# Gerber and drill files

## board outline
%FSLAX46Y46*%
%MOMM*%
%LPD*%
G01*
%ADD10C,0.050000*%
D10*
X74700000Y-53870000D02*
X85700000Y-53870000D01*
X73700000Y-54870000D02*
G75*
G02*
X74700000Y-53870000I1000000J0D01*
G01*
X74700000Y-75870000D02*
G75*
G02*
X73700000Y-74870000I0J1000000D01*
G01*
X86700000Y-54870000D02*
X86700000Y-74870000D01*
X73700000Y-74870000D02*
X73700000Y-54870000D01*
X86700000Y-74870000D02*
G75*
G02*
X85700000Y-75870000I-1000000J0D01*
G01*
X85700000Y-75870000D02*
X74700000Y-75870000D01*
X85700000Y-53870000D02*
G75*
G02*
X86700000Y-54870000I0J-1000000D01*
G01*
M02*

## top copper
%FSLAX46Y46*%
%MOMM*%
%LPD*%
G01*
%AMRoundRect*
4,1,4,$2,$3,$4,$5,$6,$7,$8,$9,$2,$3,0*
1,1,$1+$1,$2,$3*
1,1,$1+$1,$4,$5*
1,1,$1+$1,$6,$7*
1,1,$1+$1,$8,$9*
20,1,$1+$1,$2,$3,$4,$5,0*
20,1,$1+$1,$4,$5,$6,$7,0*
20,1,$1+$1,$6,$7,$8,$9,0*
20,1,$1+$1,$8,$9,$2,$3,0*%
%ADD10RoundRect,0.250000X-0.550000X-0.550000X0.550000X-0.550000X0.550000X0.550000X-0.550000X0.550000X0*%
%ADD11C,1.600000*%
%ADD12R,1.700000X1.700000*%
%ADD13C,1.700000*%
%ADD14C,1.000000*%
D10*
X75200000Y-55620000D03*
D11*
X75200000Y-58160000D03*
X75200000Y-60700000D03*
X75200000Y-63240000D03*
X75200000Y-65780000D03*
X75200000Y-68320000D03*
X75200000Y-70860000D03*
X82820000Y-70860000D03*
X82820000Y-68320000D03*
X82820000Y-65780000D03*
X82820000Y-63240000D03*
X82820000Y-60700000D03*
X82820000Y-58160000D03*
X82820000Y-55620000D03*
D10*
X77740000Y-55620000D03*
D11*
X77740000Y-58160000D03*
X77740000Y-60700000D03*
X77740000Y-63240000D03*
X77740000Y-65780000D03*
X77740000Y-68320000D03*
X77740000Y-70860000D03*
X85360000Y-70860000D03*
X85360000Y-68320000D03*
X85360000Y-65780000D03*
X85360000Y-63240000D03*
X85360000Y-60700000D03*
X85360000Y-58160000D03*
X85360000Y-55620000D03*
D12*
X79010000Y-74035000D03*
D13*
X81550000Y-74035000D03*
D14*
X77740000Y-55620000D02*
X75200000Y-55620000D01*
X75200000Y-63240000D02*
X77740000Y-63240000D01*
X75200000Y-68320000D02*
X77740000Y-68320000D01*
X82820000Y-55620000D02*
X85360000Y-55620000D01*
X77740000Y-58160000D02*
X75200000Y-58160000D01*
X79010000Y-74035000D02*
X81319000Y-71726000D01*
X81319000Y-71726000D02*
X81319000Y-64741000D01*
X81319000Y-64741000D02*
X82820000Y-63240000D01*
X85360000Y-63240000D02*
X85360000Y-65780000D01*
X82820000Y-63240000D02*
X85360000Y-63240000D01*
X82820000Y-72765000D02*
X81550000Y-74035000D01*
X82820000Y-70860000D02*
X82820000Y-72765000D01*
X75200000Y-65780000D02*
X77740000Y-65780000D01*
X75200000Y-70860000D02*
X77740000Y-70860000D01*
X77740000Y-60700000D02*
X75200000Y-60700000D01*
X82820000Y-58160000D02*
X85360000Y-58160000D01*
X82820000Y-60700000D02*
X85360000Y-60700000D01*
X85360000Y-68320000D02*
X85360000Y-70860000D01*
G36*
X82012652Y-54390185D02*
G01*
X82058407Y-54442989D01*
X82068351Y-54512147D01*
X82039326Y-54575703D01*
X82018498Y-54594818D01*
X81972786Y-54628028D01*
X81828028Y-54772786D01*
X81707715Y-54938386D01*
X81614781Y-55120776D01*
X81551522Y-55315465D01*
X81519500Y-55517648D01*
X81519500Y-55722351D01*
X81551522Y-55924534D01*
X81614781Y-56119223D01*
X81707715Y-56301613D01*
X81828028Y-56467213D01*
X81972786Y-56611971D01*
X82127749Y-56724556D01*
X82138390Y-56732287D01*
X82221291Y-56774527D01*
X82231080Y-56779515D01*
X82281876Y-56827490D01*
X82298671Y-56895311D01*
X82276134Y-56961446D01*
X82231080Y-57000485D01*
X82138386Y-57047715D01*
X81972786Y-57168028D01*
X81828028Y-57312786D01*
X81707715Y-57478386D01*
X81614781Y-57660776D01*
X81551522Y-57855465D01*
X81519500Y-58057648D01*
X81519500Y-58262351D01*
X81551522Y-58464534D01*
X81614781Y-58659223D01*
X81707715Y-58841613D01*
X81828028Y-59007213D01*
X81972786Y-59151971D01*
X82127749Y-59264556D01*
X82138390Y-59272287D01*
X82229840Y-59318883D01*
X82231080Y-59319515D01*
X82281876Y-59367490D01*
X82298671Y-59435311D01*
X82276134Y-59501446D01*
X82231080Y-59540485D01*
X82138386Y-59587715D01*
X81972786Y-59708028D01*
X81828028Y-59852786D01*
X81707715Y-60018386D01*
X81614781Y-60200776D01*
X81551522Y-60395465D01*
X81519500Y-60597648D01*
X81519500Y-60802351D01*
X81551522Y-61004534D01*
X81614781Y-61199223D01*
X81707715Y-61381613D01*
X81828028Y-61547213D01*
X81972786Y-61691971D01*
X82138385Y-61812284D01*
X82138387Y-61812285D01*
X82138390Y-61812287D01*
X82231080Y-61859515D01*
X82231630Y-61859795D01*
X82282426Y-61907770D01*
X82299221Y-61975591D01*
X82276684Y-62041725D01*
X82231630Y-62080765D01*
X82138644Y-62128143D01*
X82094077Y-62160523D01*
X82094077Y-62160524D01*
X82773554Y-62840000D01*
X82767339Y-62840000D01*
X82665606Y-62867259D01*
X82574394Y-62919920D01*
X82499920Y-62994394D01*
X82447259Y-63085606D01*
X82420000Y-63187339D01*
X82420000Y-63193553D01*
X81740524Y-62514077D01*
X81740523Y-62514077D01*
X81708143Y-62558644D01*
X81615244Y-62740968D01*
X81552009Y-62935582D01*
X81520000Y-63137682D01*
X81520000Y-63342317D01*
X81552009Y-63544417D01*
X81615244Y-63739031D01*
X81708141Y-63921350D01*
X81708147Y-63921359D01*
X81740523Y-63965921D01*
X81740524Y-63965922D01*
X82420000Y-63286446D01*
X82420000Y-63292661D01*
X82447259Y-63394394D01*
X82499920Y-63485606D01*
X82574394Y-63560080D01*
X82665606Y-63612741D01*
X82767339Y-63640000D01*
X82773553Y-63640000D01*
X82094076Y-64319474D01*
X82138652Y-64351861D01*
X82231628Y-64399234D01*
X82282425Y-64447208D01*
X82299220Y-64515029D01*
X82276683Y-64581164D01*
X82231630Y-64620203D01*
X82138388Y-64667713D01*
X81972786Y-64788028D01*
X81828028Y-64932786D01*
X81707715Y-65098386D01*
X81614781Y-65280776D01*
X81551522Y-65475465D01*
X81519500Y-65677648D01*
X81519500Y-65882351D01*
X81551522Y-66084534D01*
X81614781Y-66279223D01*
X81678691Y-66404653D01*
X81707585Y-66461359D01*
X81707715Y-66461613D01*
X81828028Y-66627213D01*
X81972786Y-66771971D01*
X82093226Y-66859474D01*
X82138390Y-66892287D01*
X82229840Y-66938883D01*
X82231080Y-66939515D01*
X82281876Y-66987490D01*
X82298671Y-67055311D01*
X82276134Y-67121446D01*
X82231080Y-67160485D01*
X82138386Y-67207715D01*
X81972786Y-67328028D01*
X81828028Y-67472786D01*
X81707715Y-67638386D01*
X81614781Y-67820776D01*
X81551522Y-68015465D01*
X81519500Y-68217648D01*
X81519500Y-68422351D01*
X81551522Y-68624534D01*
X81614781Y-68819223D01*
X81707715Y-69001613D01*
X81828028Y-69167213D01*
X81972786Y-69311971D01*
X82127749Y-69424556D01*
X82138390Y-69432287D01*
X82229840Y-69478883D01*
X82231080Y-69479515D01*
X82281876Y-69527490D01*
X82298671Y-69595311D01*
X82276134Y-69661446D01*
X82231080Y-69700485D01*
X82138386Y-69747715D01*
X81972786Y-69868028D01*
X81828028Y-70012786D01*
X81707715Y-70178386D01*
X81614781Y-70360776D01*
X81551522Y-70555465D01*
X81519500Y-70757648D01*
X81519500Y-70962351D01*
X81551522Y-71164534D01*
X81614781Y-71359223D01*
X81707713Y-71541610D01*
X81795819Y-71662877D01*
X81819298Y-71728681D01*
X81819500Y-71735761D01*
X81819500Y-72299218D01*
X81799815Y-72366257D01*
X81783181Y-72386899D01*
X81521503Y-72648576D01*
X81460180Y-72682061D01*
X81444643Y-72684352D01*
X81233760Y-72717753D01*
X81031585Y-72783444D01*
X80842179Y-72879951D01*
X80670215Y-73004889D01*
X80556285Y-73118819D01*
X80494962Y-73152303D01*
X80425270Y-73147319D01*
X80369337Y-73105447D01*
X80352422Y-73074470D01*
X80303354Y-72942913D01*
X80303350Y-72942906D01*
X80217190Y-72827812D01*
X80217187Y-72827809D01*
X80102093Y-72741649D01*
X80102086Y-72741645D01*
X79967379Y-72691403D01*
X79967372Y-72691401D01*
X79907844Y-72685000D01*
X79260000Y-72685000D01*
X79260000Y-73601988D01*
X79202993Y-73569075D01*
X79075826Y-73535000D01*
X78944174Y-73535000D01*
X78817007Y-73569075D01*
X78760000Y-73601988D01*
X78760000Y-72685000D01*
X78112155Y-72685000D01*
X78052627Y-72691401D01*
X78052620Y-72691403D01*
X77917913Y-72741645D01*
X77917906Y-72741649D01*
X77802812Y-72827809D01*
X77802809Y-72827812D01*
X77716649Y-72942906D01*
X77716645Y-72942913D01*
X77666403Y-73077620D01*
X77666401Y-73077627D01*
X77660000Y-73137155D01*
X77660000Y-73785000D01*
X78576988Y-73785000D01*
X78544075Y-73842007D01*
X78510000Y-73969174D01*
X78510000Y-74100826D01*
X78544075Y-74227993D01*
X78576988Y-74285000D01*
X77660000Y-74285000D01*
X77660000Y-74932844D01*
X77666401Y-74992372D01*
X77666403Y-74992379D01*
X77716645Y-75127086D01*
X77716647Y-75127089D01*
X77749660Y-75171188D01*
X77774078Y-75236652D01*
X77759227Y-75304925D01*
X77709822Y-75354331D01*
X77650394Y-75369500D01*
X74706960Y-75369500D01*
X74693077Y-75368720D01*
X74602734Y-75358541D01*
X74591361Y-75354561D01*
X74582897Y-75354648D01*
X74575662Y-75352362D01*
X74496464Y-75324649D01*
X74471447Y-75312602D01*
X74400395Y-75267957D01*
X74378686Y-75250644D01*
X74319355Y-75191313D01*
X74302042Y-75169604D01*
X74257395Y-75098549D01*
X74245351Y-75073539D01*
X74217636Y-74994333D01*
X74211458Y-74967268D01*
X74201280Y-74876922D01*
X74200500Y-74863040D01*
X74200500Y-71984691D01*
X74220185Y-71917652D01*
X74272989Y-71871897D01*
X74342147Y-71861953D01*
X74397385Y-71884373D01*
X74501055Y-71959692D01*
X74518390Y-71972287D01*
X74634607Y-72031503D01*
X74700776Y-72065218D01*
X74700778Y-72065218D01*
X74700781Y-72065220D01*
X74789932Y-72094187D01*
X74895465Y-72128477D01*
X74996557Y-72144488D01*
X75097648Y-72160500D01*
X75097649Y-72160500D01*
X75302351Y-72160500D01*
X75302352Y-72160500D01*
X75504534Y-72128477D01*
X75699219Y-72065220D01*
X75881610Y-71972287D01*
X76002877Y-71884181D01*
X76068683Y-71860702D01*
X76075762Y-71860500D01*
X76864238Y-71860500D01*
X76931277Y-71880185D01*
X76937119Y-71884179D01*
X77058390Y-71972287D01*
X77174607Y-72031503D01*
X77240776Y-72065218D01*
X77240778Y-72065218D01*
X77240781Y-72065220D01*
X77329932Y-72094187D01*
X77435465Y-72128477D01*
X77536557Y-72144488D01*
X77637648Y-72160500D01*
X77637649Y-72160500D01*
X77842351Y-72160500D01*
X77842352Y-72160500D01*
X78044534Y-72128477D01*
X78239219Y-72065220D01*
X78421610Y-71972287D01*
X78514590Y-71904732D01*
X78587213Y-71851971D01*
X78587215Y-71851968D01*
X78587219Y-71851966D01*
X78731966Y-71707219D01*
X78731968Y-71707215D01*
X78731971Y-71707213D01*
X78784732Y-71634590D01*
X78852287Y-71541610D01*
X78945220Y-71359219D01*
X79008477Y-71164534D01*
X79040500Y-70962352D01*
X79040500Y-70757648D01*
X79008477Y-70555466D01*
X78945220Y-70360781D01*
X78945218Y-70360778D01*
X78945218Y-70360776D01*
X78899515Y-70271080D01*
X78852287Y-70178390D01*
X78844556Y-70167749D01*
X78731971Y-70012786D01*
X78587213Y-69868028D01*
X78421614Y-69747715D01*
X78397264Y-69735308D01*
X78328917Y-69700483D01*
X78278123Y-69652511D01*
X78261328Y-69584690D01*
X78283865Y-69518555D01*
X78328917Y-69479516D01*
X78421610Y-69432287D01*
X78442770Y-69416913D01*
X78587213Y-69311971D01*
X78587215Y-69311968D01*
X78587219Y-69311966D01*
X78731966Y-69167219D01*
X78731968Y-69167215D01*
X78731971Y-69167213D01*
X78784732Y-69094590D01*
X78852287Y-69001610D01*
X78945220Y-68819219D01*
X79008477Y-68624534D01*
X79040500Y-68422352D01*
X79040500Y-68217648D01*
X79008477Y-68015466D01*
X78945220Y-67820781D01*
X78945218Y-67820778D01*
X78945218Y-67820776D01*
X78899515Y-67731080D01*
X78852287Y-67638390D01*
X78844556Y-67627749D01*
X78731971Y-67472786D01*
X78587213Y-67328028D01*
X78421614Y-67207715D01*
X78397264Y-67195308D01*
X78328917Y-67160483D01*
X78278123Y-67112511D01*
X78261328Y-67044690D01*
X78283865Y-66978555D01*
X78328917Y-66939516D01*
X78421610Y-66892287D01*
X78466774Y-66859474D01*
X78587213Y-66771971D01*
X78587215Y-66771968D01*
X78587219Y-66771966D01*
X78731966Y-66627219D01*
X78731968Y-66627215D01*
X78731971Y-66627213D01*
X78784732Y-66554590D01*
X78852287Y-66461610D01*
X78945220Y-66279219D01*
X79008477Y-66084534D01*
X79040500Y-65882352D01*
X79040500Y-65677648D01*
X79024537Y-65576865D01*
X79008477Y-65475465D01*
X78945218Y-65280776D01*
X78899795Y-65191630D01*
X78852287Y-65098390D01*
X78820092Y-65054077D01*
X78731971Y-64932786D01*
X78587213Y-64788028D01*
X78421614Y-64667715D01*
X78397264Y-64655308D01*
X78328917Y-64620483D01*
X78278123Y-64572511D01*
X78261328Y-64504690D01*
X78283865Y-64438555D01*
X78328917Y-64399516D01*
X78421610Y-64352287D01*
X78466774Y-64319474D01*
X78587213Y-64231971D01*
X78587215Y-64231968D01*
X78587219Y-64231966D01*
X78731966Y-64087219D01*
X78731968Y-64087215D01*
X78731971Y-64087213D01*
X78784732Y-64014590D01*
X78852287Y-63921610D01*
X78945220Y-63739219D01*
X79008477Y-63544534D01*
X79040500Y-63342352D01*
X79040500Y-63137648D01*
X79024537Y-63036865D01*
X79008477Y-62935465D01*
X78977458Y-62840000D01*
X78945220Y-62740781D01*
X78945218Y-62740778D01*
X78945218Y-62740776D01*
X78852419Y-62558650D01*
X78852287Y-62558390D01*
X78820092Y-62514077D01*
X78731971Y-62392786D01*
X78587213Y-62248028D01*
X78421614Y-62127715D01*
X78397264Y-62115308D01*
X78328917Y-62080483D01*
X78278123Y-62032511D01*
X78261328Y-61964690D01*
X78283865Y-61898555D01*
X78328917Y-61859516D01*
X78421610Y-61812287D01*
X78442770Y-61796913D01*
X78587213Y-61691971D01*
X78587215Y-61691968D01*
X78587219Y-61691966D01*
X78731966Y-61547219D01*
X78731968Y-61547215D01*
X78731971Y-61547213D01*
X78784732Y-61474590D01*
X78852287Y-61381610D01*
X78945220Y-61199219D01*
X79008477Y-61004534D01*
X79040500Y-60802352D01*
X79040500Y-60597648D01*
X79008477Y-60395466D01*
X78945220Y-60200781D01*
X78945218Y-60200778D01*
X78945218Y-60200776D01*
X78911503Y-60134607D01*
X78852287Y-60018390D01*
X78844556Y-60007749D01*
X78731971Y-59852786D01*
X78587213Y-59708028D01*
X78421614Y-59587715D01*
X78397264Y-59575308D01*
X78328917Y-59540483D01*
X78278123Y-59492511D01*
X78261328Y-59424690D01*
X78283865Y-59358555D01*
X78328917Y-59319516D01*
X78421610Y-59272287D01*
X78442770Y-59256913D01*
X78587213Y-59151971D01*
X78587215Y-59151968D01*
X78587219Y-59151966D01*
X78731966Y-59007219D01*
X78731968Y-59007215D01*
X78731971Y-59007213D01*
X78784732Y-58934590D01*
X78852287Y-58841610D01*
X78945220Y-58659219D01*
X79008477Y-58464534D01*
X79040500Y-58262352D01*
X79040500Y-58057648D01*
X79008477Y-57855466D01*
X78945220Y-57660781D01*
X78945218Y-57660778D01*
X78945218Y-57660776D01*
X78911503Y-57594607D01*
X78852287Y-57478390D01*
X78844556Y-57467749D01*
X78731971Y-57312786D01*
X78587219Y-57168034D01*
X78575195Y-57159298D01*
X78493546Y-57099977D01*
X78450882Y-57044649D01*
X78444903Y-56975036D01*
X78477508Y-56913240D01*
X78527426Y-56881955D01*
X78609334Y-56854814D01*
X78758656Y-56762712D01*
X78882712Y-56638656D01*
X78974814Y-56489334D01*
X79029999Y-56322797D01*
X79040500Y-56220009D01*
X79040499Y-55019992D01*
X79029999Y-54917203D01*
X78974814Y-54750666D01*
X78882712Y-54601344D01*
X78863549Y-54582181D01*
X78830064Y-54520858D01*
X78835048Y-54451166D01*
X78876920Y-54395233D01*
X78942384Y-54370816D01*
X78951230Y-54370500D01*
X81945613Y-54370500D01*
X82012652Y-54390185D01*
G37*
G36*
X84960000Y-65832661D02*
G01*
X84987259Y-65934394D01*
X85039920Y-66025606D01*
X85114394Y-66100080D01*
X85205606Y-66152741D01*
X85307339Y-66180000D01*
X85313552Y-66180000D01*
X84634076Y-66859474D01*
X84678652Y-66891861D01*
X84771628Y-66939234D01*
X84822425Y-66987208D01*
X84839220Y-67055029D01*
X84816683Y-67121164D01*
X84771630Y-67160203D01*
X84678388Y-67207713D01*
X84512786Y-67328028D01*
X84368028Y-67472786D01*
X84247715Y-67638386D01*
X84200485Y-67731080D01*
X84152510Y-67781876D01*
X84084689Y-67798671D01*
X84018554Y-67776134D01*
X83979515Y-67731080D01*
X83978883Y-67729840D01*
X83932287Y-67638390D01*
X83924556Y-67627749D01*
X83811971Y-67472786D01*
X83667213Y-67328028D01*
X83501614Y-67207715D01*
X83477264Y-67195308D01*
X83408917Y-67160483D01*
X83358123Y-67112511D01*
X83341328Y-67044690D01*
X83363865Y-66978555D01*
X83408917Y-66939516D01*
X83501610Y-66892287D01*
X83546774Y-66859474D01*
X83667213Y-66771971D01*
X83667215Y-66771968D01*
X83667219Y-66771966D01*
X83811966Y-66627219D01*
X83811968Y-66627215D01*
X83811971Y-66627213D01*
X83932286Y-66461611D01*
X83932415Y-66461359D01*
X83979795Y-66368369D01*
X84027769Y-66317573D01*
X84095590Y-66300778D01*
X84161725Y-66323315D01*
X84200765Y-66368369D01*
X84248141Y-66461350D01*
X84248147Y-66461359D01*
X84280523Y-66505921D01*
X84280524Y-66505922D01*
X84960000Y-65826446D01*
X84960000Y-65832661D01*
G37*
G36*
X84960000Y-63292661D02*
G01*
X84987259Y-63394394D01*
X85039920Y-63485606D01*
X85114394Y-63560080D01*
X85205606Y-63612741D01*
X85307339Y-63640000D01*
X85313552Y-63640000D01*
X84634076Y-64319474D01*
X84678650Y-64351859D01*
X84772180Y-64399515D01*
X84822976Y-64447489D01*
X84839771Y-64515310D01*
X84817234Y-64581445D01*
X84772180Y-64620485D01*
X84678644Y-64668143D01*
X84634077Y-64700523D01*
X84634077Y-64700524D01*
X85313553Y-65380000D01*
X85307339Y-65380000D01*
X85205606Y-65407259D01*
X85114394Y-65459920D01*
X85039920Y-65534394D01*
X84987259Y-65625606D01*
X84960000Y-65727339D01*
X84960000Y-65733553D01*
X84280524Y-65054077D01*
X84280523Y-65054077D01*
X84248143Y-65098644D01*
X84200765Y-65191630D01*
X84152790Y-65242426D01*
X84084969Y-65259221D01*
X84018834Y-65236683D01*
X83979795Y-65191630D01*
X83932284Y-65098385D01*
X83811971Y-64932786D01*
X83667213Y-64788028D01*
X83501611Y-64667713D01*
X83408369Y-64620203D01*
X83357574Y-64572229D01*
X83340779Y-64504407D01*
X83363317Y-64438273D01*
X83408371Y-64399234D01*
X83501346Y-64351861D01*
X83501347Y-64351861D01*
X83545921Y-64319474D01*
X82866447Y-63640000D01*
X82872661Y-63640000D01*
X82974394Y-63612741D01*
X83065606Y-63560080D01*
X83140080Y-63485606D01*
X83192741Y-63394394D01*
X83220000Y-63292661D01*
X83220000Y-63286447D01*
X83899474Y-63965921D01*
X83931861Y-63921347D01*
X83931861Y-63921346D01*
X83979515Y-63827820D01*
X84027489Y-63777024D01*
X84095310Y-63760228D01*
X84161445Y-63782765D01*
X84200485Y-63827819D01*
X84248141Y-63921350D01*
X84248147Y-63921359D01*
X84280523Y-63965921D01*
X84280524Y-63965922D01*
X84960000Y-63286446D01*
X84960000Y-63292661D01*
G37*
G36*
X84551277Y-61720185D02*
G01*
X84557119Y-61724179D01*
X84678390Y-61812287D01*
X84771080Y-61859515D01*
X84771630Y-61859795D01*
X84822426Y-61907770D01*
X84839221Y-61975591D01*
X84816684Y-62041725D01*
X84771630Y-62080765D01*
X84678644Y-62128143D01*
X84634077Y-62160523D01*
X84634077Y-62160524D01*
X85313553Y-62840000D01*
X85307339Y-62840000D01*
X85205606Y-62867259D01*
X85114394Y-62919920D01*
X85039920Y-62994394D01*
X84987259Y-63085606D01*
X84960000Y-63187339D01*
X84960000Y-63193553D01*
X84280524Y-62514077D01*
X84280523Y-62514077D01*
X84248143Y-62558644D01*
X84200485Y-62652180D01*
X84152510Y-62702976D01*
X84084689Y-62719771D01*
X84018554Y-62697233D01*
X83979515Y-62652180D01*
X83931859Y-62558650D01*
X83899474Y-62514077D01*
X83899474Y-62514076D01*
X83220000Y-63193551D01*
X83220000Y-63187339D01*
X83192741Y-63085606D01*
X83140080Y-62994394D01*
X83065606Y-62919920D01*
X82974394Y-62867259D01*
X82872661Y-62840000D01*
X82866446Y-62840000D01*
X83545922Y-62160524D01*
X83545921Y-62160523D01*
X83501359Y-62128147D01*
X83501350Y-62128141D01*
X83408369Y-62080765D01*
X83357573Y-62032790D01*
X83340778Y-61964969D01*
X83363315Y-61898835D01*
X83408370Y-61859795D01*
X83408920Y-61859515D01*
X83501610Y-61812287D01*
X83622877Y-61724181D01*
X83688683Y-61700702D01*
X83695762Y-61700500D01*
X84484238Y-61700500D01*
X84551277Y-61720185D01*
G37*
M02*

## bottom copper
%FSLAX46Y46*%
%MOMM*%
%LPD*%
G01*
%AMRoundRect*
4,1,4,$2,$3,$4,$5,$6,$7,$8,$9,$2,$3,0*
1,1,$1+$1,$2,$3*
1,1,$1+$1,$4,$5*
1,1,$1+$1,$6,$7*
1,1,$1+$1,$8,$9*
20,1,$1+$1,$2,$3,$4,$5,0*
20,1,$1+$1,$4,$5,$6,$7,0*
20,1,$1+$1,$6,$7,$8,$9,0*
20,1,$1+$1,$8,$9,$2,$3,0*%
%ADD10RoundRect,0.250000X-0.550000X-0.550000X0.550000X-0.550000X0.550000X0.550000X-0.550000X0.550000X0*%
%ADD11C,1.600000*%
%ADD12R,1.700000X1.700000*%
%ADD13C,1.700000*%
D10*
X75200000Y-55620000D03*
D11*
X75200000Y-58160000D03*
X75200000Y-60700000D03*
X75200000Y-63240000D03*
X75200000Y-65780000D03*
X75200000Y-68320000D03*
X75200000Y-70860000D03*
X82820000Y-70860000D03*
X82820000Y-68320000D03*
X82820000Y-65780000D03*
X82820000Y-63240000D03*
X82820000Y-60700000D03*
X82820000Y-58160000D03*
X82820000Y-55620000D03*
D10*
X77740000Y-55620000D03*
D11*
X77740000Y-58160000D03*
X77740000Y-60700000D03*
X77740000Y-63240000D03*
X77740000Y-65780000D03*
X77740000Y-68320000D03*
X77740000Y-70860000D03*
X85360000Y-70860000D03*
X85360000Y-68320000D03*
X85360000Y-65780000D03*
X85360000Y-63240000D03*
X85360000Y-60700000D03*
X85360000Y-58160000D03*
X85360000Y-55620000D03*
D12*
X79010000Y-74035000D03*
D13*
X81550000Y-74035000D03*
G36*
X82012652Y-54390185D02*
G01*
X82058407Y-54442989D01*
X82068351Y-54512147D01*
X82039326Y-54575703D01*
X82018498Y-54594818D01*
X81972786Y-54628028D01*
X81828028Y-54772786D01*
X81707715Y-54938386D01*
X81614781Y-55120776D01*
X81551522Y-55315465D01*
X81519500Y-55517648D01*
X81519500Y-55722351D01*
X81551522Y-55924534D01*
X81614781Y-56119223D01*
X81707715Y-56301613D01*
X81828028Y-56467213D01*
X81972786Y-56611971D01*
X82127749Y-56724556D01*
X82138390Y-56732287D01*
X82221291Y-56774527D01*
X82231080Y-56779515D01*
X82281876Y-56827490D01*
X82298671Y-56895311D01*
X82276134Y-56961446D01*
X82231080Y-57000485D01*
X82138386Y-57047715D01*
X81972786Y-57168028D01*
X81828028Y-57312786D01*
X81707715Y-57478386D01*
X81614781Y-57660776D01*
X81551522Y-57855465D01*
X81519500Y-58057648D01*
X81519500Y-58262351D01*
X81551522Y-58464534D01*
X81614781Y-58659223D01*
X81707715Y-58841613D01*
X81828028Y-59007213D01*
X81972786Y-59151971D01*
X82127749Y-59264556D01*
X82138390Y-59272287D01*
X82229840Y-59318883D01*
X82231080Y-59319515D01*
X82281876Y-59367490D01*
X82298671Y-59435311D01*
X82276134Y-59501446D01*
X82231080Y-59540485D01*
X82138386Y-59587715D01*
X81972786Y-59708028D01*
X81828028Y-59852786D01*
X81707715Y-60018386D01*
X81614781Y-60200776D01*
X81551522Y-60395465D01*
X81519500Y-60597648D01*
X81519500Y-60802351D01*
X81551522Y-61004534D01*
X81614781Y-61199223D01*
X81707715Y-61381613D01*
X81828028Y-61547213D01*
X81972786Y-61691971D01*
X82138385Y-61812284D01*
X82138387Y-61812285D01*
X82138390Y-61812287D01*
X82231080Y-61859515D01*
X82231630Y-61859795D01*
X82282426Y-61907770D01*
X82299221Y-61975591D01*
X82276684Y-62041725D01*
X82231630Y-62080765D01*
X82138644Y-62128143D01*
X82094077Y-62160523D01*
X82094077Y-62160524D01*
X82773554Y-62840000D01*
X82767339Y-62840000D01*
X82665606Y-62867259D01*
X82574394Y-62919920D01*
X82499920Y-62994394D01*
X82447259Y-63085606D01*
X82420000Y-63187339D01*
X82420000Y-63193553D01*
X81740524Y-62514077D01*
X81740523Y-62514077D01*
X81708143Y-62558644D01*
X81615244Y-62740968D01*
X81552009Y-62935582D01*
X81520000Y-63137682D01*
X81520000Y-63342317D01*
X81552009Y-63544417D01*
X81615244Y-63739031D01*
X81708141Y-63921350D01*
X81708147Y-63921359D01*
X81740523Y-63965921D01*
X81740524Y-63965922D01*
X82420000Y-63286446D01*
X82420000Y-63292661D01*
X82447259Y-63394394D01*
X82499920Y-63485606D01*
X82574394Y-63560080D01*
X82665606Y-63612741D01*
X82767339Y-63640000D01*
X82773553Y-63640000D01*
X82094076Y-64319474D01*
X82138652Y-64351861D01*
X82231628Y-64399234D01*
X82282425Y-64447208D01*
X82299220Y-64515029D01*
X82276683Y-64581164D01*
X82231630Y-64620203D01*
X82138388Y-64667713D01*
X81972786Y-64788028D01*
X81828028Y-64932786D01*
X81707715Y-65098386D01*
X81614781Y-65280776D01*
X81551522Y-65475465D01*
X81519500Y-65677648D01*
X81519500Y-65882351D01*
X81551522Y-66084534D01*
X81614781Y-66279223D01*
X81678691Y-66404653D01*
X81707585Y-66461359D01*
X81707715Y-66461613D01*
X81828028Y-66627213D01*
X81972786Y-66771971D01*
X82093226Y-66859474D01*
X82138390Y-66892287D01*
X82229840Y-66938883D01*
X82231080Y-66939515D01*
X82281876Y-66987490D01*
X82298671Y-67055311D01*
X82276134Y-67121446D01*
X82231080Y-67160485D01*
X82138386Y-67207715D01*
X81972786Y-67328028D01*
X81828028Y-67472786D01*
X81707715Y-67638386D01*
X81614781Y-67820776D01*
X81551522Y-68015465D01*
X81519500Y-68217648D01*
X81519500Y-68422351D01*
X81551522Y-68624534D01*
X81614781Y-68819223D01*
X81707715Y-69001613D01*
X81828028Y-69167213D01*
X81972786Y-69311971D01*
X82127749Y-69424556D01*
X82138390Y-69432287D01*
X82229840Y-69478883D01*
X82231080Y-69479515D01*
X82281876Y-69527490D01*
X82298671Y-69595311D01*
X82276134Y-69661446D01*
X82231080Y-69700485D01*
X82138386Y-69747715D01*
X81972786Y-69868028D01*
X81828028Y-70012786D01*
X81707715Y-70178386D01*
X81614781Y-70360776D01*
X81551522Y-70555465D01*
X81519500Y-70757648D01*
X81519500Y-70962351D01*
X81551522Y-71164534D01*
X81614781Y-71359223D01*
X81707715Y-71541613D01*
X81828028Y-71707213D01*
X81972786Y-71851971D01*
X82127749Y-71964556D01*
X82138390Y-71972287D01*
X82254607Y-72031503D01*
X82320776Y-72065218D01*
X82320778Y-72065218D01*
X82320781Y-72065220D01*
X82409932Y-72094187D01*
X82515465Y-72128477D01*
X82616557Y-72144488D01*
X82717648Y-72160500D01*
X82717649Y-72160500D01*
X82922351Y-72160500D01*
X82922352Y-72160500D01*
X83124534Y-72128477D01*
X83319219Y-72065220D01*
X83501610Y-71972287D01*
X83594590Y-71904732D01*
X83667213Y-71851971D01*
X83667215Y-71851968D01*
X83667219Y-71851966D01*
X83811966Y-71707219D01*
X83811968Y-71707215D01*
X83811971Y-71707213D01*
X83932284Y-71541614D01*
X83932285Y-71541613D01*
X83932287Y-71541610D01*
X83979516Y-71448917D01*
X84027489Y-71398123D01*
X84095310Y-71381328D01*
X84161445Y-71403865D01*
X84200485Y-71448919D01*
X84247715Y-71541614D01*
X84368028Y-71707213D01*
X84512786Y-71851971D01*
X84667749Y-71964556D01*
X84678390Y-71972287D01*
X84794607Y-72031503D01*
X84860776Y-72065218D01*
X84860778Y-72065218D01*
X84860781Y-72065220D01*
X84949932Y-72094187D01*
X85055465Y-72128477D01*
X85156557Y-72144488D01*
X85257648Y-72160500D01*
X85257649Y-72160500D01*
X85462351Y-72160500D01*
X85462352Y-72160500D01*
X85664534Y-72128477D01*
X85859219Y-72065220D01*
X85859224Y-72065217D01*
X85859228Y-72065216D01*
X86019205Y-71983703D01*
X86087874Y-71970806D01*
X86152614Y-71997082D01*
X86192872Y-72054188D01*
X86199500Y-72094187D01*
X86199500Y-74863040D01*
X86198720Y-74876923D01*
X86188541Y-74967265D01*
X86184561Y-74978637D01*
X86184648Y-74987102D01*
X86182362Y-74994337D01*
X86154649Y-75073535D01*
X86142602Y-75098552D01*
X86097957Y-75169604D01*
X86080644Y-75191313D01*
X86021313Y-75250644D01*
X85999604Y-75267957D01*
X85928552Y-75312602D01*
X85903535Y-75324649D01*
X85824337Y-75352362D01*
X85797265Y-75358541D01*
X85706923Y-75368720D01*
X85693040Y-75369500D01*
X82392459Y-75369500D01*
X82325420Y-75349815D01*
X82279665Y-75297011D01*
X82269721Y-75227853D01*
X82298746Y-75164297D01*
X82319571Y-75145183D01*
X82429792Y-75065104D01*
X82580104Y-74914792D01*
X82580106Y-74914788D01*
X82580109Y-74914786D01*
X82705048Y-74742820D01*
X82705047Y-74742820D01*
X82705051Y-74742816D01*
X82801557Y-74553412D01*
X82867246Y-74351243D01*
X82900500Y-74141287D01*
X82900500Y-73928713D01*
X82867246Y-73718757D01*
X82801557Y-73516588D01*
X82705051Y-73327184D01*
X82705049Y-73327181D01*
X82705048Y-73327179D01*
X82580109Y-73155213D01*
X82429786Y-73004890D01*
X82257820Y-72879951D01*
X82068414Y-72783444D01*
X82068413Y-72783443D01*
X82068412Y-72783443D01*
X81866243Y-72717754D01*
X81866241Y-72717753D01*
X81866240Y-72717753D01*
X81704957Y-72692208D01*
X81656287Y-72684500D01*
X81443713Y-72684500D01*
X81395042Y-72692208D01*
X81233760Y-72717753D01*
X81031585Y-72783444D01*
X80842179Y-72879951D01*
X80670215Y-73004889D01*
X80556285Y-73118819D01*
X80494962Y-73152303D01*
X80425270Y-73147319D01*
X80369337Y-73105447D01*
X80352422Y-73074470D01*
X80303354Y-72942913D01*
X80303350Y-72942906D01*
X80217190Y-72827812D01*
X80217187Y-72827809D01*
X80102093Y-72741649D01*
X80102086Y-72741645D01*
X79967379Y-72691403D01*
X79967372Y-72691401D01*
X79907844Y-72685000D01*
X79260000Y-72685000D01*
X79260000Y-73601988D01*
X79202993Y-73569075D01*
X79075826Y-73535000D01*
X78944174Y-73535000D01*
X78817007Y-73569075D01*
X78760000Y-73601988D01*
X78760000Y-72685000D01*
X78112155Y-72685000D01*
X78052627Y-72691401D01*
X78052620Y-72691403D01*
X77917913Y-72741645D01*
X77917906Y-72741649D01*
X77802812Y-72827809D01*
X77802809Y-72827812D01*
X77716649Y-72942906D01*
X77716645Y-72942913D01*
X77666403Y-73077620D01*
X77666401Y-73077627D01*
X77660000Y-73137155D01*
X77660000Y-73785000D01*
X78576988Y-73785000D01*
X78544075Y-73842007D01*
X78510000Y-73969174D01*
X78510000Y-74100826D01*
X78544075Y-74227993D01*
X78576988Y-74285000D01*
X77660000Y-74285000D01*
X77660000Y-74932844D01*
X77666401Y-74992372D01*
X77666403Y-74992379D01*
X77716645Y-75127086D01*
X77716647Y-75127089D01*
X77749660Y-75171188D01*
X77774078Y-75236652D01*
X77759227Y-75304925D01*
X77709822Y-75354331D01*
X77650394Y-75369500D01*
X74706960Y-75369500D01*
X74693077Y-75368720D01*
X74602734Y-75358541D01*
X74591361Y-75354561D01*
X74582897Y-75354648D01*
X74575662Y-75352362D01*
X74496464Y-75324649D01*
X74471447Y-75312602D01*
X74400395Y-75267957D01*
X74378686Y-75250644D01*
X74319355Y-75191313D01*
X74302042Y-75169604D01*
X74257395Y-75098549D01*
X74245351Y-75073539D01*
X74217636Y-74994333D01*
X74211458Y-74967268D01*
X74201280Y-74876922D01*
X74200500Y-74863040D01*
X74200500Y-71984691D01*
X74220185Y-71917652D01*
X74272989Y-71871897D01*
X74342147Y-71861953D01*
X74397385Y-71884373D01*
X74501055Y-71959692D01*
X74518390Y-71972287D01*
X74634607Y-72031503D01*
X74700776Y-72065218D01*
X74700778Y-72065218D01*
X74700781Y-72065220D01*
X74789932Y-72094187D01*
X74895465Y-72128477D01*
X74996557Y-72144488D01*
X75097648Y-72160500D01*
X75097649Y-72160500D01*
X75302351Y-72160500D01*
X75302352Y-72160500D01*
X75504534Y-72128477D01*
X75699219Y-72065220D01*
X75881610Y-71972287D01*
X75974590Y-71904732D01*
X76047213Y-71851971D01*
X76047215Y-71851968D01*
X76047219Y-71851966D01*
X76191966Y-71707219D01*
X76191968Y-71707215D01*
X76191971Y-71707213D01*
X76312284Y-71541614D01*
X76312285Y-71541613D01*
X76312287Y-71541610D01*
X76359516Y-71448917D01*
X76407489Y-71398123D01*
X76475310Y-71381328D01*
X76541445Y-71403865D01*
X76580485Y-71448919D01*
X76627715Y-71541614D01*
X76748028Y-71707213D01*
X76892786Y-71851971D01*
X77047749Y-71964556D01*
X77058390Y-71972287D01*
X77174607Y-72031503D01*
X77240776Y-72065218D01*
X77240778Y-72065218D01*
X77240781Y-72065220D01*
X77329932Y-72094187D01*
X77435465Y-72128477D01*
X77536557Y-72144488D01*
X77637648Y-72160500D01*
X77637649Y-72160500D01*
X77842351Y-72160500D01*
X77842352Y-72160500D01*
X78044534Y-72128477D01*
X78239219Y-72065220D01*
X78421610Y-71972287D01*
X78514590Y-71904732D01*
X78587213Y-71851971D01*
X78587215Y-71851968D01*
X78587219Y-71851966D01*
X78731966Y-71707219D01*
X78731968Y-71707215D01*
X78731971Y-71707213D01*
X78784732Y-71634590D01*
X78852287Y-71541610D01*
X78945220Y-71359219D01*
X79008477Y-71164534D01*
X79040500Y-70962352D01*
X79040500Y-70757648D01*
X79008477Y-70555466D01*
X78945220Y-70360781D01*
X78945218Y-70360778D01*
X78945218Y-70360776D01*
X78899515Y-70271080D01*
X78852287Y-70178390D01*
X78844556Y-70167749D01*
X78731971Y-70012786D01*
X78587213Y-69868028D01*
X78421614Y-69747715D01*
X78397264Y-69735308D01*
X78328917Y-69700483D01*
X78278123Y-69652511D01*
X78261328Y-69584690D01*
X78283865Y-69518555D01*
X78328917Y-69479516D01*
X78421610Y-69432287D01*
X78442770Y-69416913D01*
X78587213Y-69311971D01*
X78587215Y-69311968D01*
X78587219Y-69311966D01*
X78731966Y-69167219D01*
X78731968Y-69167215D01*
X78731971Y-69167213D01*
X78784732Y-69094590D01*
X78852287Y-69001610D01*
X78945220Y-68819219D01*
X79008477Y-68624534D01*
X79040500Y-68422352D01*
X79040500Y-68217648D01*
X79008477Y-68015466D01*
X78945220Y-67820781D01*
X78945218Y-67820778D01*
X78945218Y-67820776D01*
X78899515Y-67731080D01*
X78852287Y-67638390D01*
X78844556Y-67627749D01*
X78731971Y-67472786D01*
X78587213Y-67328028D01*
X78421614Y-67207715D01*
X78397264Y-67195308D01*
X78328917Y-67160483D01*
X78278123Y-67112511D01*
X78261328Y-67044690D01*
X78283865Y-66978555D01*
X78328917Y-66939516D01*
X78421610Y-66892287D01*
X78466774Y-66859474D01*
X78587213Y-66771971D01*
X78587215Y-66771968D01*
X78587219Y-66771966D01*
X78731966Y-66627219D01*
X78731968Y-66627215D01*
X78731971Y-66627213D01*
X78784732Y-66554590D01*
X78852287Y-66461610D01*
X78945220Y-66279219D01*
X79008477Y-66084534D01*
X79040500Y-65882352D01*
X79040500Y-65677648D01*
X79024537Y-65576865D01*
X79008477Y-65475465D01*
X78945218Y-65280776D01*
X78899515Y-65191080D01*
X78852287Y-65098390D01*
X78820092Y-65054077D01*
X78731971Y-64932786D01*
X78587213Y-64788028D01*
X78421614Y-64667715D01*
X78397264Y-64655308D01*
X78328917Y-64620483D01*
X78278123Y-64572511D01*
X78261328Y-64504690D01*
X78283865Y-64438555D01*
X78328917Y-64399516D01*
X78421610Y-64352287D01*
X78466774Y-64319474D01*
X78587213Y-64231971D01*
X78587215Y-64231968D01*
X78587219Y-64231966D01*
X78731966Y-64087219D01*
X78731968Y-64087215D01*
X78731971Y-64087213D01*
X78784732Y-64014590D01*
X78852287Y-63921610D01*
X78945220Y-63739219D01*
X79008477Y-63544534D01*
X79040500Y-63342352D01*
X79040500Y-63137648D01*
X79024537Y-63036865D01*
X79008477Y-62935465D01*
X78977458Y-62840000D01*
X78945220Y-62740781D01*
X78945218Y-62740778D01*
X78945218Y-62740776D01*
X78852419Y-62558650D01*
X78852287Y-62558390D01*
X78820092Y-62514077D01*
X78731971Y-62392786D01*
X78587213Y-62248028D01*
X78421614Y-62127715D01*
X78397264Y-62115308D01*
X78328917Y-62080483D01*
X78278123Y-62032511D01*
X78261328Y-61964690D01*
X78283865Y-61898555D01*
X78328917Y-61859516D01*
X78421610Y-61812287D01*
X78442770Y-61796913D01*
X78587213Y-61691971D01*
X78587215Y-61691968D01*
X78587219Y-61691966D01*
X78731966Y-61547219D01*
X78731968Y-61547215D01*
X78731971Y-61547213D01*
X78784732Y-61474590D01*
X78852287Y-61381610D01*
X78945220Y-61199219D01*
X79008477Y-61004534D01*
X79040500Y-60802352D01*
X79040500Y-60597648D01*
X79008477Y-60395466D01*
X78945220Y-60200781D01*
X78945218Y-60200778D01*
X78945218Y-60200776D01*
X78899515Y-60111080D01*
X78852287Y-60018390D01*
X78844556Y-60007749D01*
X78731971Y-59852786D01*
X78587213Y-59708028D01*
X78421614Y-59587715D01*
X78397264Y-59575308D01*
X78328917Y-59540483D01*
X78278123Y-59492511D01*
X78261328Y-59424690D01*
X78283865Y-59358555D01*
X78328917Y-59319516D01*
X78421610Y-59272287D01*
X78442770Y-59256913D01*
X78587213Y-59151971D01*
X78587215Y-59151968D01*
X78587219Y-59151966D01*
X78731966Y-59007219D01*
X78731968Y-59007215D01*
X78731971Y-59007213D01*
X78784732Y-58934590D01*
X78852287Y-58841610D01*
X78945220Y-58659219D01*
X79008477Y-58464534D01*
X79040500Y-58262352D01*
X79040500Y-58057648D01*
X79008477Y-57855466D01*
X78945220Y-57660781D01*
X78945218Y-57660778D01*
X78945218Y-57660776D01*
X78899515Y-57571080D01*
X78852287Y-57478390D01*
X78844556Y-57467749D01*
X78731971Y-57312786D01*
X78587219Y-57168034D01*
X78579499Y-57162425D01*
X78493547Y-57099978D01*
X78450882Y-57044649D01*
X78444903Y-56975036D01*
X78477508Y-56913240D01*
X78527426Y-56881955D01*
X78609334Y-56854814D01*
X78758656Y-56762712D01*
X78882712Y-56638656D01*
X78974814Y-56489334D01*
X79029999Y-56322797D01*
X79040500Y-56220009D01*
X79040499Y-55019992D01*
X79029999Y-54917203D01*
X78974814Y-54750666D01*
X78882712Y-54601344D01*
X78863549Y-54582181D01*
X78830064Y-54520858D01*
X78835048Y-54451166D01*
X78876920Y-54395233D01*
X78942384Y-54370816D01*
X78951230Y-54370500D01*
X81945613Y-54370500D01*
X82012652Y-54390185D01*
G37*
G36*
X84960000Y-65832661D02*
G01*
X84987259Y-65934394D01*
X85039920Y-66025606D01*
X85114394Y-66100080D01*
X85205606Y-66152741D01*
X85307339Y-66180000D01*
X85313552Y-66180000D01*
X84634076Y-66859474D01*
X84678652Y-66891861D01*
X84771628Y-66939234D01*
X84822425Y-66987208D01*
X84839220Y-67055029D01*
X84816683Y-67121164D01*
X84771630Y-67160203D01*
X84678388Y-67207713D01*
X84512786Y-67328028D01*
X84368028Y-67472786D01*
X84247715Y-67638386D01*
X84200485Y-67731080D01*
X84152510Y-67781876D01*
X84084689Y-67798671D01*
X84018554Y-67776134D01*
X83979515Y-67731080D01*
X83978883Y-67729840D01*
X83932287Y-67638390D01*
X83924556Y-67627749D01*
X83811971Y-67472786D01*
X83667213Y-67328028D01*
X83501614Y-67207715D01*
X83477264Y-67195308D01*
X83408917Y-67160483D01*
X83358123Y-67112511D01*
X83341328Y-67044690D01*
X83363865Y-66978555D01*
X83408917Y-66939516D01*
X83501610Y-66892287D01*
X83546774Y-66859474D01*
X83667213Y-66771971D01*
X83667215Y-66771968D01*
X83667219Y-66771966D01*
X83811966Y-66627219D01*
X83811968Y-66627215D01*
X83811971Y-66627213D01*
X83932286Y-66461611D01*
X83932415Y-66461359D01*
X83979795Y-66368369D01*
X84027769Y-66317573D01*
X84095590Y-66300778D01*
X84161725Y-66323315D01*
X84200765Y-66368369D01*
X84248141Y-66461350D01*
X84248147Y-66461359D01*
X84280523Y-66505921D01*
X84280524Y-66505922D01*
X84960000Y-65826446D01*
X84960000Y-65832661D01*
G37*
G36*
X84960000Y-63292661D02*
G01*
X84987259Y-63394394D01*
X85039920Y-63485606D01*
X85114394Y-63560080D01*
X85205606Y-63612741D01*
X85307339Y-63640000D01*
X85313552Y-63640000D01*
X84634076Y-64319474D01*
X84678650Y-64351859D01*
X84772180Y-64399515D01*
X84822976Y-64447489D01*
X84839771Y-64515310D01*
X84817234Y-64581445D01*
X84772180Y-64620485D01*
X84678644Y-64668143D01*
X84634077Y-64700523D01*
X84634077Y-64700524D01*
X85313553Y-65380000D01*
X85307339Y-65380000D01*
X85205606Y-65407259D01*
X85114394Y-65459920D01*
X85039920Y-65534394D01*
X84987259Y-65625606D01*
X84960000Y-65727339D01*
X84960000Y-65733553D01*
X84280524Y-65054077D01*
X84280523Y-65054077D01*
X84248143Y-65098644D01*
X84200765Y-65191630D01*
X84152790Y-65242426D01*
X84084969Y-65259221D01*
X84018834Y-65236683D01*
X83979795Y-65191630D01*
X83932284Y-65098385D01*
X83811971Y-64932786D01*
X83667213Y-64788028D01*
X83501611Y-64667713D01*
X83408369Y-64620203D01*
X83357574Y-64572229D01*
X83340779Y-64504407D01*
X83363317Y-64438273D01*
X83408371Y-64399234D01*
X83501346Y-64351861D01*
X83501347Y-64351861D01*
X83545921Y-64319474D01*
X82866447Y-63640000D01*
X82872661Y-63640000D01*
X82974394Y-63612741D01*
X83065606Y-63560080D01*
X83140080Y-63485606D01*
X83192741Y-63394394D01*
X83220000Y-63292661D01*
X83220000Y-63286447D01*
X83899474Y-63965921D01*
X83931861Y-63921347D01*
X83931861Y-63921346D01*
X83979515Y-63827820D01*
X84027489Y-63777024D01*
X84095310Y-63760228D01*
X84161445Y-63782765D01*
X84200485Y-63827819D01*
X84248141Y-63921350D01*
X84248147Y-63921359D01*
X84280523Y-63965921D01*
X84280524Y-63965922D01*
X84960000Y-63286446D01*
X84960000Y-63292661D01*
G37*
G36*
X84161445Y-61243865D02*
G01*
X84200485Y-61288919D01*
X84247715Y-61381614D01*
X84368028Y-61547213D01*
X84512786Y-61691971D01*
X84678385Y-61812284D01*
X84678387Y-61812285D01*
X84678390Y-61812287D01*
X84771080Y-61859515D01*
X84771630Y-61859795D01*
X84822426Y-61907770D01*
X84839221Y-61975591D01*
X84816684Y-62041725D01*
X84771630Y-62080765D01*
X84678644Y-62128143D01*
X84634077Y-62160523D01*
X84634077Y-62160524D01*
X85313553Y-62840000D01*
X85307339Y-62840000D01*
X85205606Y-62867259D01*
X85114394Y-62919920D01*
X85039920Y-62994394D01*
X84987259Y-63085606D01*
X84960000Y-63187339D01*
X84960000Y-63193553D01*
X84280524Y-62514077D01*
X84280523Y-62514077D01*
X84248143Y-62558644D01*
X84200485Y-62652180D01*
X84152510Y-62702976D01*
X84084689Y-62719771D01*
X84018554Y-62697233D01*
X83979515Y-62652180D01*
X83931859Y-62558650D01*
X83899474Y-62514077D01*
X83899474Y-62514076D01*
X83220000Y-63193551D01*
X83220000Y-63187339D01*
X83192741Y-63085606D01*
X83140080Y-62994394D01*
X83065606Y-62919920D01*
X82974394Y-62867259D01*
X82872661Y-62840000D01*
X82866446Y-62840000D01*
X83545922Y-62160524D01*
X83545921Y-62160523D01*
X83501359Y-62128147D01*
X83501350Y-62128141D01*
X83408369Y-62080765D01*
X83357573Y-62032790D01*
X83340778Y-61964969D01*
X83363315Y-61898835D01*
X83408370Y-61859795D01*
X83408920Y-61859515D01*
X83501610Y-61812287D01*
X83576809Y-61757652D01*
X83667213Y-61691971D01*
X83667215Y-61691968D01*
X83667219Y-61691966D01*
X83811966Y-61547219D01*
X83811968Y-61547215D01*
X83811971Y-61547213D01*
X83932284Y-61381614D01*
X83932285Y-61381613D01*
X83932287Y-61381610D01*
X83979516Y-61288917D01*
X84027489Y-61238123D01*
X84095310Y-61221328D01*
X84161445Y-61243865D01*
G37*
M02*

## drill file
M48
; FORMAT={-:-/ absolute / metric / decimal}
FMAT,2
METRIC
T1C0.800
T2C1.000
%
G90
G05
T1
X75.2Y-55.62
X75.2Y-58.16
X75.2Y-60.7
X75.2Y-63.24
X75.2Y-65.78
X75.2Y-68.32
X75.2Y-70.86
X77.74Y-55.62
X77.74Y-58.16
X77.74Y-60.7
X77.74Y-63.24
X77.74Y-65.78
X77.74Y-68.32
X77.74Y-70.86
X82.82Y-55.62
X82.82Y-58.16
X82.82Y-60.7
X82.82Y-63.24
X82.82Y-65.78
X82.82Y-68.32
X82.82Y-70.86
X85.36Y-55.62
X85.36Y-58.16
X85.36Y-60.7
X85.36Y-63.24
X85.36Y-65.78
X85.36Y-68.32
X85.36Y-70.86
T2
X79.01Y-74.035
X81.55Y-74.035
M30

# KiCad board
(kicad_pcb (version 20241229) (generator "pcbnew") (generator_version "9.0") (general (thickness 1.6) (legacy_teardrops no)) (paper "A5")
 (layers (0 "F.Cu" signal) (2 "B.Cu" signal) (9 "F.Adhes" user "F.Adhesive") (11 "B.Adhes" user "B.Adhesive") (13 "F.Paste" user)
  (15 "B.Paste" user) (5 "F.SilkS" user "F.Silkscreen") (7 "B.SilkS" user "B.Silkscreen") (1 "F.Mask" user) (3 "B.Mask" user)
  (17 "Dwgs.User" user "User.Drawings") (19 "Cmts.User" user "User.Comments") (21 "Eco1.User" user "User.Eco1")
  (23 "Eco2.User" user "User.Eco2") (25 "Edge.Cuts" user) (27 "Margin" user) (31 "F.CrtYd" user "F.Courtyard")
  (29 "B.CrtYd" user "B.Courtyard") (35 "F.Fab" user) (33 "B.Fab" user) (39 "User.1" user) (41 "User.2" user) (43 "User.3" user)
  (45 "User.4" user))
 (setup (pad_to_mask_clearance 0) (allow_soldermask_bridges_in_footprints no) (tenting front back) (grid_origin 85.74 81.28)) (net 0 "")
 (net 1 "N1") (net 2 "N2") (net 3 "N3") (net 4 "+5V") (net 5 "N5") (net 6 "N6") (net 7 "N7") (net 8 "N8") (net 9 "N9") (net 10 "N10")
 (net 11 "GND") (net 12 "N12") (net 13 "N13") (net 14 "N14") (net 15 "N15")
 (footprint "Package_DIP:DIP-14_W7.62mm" (layer "F.Cu") (at 75.2 55.62)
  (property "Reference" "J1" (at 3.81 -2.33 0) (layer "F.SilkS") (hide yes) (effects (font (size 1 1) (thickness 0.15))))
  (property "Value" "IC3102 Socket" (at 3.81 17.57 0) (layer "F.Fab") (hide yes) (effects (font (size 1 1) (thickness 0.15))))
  (pad "1" thru_hole roundrect (at 0 0) (size 1.6 1.6) (drill 0.8) (layers "*.Cu" "*.Mask") (remove_unused_layers no)
   (roundrect_rratio 0.15625) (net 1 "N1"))
  (pad "2" thru_hole circle (at 0 2.54) (size 1.6 1.6) (drill 0.8) (layers "*.Cu" "*.Mask") (remove_unused_layers no) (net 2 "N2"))
  (pad "3" thru_hole circle (at 0 5.08) (size 1.6 1.6) (drill 0.8) (layers "*.Cu" "*.Mask") (remove_unused_layers no) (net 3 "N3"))
  (pad "4" thru_hole circle (at 0 7.62) (size 1.6 1.6) (drill 0.8) (layers "*.Cu" "*.Mask") (remove_unused_layers no) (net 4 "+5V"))
  (pad "5" thru_hole circle (at 0 10.16) (size 1.6 1.6) (drill 0.8) (layers "*.Cu" "*.Mask") (remove_unused_layers no) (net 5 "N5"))
  (pad "6" thru_hole circle (at 0 12.7) (size 1.6 1.6) (drill 0.8) (layers "*.Cu" "*.Mask") (remove_unused_layers no) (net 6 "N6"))
  (pad "7" thru_hole circle (at 0 15.24) (size 1.6 1.6) (drill 0.8) (layers "*.Cu" "*.Mask") (remove_unused_layers no) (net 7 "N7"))
  (pad "8" thru_hole circle (at 7.62 15.24) (size 1.6 1.6) (drill 0.8) (layers "*.Cu" "*.Mask") (remove_unused_layers no) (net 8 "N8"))
  (pad "9" thru_hole circle (at 7.62 12.7) (size 1.6 1.6) (drill 0.8) (layers "*.Cu" "*.Mask") (remove_unused_layers no) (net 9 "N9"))
  (pad "10" thru_hole circle (at 7.62 10.16) (size 1.6 1.6) (drill 0.8) (layers "*.Cu" "*.Mask") (remove_unused_layers no) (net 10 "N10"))
  (pad "11" thru_hole circle (at 7.62 7.62) (size 1.6 1.6) (drill 0.8) (layers "*.Cu" "*.Mask") (remove_unused_layers no) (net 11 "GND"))
  (pad "12" thru_hole circle (at 7.62 5.08) (size 1.6 1.6) (drill 0.8) (layers "*.Cu" "*.Mask") (remove_unused_layers no) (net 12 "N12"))
  (pad "13" thru_hole circle (at 7.62 2.54) (size 1.6 1.6) (drill 0.8) (layers "*.Cu" "*.Mask") (remove_unused_layers no) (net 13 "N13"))
  (pad "14" thru_hole circle (at 7.62 0) (size 1.6 1.6) (drill 0.8) (layers "*.Cu" "*.Mask") (remove_unused_layers no) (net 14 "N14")))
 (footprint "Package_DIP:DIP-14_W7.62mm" (layer "F.Cu") (at 77.74 55.62)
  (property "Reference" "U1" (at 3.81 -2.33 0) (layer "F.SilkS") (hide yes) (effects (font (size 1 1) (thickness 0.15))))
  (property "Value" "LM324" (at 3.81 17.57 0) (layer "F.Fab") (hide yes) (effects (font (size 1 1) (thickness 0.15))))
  (pad "1" thru_hole roundrect (at 0 0) (size 1.6 1.6) (drill 0.8) (layers "*.Cu" "*.Mask") (remove_unused_layers no)
   (roundrect_rratio 0.15625) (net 1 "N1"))
  (pad "2" thru_hole circle (at 0 2.54) (size 1.6 1.6) (drill 0.8) (layers "*.Cu" "*.Mask") (remove_unused_layers no) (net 2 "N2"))
  (pad "3" thru_hole circle (at 0 5.08) (size 1.6 1.6) (drill 0.8) (layers "*.Cu" "*.Mask") (remove_unused_layers no) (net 3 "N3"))
  (pad "4" thru_hole circle (at 0 7.62) (size 1.6 1.6) (drill 0.8) (layers "*.Cu" "*.Mask") (remove_unused_layers no) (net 4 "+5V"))
  (pad "5" thru_hole circle (at 0 10.16) (size 1.6 1.6) (drill 0.8) (layers "*.Cu" "*.Mask") (remove_unused_layers no) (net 5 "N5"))
  (pad "6" thru_hole circle (at 0 12.7) (size 1.6 1.6) (drill 0.8) (layers "*.Cu" "*.Mask") (remove_unused_layers no) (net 6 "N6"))
  (pad "7" thru_hole circle (at 0 15.24) (size 1.6 1.6) (drill 0.8) (layers "*.Cu" "*.Mask") (remove_unused_layers no) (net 7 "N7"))
  (pad "8" thru_hole circle (at 7.62 15.24) (size 1.6 1.6) (drill 0.8) (layers "*.Cu" "*.Mask") (remove_unused_layers no) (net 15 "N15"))
  (pad "9" thru_hole circle (at 7.62 12.7) (size 1.6 1.6) (drill 0.8) (layers "*.Cu" "*.Mask") (remove_unused_layers no) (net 15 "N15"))
  (pad "10" thru_hole circle (at 7.62 10.16) (size 1.6 1.6) (drill 0.8) (layers "*.Cu" "*.Mask") (remove_unused_layers no) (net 11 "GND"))
  (pad "11" thru_hole circle (at 7.62 7.62) (size 1.6 1.6) (drill 0.8) (layers "*.Cu" "*.Mask") (remove_unused_layers no) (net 11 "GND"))
  (pad "12" thru_hole circle (at 7.62 5.08) (size 1.6 1.6) (drill 0.8) (layers "*.Cu" "*.Mask") (remove_unused_layers no) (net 12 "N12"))
  (pad "13" thru_hole circle (at 7.62 2.54) (size 1.6 1.6) (drill 0.8) (layers "*.Cu" "*.Mask") (remove_unused_layers no) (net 13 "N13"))
  (pad "14" thru_hole circle (at 7.62 0) (size 1.6 1.6) (drill 0.8) (layers "*.Cu" "*.Mask") (remove_unused_layers no) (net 14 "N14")))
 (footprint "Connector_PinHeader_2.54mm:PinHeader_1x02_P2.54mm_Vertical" (layer "F.Cu") (at 79.01 74.035 90)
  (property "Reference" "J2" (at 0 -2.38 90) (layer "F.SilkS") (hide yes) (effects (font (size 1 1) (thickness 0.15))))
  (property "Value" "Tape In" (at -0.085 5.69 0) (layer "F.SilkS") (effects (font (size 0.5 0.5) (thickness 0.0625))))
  (pad "1" thru_hole rect (at 0 0 90) (size 1.7 1.7) (drill 1) (layers "*.Cu" "*.Mask") (remove_unused_layers no) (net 11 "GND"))
  (pad "2" thru_hole circle (at 0 2.54 90) (size 1.7 1.7) (drill 1) (layers "*.Cu" "*.Mask") (remove_unused_layers no) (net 8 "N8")))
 (gr_line (start 74.7 53.87) (end 85.7 53.87) (stroke (width 0.05) (type default)) (layer "Edge.Cuts"))
 (gr_arc (start 73.7 54.87) (mid 73.992893 54.162893) (end 74.7 53.87) (stroke (width 0.05) (type default)) (layer "Edge.Cuts"))
 (gr_arc (start 74.7 75.87) (mid 73.992893 75.577107) (end 73.7 74.87) (stroke (width 0.05) (type default)) (layer "Edge.Cuts"))
 (gr_line (start 86.7 54.87) (end 86.7 74.87) (stroke (width 0.05) (type default)) (layer "Edge.Cuts"))
 (gr_line (start 73.7 74.87) (end 73.7 54.87) (stroke (width 0.05) (type default)) (layer "Edge.Cuts"))
 (gr_arc (start 86.7 74.87) (mid 86.407107 75.577107) (end 85.7 75.87) (stroke (width 0.05) (type default)) (layer "Edge.Cuts"))
 (gr_line (start 85.7 75.87) (end 74.7 75.87) (stroke (width 0.05) (type default)) (layer "Edge.Cuts"))
 (gr_arc (start 85.7 53.87) (mid 86.407107 54.162893) (end 86.7 54.87) (stroke (width 0.05) (type default)) (layer "Edge.Cuts"))
 (segment (start 77.74 55.62) (end 75.2 55.62) (width 1) (layer "F.Cu") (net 1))
 (segment (start 75.2 63.24) (end 77.74 63.24) (width 1) (layer "F.Cu") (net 4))
 (segment (start 75.2 68.32) (end 77.74 68.32) (width 1) (layer "F.Cu") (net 6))
 (segment (start 82.82 55.62) (end 85.36 55.62) (width 1) (layer "F.Cu") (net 14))
 (segment (start 77.74 58.16) (end 75.2 58.16) (width 1) (layer "F.Cu") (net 2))
 (segment (start 79.01 74.035) (end 81.319 71.726) (width 1) (layer "F.Cu") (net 11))
 (segment (start 81.319 71.726) (end 81.319 64.741) (width 1) (layer "F.Cu") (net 11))
 (segment (start 81.319 64.741) (end 82.82 63.24) (width 1) (layer "F.Cu") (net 11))
 (segment (start 85.36 63.24) (end 85.36 65.78) (width 1) (layer "F.Cu") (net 11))
 (segment (start 82.82 63.24) (end 85.36 63.24) (width 1) (layer "F.Cu") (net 11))
 (segment (start 82.82 72.765) (end 81.55 74.035) (width 1) (layer "F.Cu") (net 8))
 (segment (start 82.82 70.86) (end 82.82 72.765) (width 1) (layer "F.Cu") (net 8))
 (segment (start 75.2 65.78) (end 77.74 65.78) (width 1) (layer "F.Cu") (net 5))
 (segment (start 75.2 70.86) (end 77.74 70.86) (width 1) (layer "F.Cu") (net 7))
 (segment (start 77.74 60.7) (end 75.2 60.7) (width 1) (layer "F.Cu") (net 3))
 (segment (start 82.82 58.16) (end 85.36 58.16) (width 1) (layer "F.Cu") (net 13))
 (segment (start 82.82 60.7) (end 85.36 60.7) (width 1) (layer "F.Cu") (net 12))
 (segment (start 85.36 68.32) (end 85.36 70.86) (width 1) (layer "F.Cu") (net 15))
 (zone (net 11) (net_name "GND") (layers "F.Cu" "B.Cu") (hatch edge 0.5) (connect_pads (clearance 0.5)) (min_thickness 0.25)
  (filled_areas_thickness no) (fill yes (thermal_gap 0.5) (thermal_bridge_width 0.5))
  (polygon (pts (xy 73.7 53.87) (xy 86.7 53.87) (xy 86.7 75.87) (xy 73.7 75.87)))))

